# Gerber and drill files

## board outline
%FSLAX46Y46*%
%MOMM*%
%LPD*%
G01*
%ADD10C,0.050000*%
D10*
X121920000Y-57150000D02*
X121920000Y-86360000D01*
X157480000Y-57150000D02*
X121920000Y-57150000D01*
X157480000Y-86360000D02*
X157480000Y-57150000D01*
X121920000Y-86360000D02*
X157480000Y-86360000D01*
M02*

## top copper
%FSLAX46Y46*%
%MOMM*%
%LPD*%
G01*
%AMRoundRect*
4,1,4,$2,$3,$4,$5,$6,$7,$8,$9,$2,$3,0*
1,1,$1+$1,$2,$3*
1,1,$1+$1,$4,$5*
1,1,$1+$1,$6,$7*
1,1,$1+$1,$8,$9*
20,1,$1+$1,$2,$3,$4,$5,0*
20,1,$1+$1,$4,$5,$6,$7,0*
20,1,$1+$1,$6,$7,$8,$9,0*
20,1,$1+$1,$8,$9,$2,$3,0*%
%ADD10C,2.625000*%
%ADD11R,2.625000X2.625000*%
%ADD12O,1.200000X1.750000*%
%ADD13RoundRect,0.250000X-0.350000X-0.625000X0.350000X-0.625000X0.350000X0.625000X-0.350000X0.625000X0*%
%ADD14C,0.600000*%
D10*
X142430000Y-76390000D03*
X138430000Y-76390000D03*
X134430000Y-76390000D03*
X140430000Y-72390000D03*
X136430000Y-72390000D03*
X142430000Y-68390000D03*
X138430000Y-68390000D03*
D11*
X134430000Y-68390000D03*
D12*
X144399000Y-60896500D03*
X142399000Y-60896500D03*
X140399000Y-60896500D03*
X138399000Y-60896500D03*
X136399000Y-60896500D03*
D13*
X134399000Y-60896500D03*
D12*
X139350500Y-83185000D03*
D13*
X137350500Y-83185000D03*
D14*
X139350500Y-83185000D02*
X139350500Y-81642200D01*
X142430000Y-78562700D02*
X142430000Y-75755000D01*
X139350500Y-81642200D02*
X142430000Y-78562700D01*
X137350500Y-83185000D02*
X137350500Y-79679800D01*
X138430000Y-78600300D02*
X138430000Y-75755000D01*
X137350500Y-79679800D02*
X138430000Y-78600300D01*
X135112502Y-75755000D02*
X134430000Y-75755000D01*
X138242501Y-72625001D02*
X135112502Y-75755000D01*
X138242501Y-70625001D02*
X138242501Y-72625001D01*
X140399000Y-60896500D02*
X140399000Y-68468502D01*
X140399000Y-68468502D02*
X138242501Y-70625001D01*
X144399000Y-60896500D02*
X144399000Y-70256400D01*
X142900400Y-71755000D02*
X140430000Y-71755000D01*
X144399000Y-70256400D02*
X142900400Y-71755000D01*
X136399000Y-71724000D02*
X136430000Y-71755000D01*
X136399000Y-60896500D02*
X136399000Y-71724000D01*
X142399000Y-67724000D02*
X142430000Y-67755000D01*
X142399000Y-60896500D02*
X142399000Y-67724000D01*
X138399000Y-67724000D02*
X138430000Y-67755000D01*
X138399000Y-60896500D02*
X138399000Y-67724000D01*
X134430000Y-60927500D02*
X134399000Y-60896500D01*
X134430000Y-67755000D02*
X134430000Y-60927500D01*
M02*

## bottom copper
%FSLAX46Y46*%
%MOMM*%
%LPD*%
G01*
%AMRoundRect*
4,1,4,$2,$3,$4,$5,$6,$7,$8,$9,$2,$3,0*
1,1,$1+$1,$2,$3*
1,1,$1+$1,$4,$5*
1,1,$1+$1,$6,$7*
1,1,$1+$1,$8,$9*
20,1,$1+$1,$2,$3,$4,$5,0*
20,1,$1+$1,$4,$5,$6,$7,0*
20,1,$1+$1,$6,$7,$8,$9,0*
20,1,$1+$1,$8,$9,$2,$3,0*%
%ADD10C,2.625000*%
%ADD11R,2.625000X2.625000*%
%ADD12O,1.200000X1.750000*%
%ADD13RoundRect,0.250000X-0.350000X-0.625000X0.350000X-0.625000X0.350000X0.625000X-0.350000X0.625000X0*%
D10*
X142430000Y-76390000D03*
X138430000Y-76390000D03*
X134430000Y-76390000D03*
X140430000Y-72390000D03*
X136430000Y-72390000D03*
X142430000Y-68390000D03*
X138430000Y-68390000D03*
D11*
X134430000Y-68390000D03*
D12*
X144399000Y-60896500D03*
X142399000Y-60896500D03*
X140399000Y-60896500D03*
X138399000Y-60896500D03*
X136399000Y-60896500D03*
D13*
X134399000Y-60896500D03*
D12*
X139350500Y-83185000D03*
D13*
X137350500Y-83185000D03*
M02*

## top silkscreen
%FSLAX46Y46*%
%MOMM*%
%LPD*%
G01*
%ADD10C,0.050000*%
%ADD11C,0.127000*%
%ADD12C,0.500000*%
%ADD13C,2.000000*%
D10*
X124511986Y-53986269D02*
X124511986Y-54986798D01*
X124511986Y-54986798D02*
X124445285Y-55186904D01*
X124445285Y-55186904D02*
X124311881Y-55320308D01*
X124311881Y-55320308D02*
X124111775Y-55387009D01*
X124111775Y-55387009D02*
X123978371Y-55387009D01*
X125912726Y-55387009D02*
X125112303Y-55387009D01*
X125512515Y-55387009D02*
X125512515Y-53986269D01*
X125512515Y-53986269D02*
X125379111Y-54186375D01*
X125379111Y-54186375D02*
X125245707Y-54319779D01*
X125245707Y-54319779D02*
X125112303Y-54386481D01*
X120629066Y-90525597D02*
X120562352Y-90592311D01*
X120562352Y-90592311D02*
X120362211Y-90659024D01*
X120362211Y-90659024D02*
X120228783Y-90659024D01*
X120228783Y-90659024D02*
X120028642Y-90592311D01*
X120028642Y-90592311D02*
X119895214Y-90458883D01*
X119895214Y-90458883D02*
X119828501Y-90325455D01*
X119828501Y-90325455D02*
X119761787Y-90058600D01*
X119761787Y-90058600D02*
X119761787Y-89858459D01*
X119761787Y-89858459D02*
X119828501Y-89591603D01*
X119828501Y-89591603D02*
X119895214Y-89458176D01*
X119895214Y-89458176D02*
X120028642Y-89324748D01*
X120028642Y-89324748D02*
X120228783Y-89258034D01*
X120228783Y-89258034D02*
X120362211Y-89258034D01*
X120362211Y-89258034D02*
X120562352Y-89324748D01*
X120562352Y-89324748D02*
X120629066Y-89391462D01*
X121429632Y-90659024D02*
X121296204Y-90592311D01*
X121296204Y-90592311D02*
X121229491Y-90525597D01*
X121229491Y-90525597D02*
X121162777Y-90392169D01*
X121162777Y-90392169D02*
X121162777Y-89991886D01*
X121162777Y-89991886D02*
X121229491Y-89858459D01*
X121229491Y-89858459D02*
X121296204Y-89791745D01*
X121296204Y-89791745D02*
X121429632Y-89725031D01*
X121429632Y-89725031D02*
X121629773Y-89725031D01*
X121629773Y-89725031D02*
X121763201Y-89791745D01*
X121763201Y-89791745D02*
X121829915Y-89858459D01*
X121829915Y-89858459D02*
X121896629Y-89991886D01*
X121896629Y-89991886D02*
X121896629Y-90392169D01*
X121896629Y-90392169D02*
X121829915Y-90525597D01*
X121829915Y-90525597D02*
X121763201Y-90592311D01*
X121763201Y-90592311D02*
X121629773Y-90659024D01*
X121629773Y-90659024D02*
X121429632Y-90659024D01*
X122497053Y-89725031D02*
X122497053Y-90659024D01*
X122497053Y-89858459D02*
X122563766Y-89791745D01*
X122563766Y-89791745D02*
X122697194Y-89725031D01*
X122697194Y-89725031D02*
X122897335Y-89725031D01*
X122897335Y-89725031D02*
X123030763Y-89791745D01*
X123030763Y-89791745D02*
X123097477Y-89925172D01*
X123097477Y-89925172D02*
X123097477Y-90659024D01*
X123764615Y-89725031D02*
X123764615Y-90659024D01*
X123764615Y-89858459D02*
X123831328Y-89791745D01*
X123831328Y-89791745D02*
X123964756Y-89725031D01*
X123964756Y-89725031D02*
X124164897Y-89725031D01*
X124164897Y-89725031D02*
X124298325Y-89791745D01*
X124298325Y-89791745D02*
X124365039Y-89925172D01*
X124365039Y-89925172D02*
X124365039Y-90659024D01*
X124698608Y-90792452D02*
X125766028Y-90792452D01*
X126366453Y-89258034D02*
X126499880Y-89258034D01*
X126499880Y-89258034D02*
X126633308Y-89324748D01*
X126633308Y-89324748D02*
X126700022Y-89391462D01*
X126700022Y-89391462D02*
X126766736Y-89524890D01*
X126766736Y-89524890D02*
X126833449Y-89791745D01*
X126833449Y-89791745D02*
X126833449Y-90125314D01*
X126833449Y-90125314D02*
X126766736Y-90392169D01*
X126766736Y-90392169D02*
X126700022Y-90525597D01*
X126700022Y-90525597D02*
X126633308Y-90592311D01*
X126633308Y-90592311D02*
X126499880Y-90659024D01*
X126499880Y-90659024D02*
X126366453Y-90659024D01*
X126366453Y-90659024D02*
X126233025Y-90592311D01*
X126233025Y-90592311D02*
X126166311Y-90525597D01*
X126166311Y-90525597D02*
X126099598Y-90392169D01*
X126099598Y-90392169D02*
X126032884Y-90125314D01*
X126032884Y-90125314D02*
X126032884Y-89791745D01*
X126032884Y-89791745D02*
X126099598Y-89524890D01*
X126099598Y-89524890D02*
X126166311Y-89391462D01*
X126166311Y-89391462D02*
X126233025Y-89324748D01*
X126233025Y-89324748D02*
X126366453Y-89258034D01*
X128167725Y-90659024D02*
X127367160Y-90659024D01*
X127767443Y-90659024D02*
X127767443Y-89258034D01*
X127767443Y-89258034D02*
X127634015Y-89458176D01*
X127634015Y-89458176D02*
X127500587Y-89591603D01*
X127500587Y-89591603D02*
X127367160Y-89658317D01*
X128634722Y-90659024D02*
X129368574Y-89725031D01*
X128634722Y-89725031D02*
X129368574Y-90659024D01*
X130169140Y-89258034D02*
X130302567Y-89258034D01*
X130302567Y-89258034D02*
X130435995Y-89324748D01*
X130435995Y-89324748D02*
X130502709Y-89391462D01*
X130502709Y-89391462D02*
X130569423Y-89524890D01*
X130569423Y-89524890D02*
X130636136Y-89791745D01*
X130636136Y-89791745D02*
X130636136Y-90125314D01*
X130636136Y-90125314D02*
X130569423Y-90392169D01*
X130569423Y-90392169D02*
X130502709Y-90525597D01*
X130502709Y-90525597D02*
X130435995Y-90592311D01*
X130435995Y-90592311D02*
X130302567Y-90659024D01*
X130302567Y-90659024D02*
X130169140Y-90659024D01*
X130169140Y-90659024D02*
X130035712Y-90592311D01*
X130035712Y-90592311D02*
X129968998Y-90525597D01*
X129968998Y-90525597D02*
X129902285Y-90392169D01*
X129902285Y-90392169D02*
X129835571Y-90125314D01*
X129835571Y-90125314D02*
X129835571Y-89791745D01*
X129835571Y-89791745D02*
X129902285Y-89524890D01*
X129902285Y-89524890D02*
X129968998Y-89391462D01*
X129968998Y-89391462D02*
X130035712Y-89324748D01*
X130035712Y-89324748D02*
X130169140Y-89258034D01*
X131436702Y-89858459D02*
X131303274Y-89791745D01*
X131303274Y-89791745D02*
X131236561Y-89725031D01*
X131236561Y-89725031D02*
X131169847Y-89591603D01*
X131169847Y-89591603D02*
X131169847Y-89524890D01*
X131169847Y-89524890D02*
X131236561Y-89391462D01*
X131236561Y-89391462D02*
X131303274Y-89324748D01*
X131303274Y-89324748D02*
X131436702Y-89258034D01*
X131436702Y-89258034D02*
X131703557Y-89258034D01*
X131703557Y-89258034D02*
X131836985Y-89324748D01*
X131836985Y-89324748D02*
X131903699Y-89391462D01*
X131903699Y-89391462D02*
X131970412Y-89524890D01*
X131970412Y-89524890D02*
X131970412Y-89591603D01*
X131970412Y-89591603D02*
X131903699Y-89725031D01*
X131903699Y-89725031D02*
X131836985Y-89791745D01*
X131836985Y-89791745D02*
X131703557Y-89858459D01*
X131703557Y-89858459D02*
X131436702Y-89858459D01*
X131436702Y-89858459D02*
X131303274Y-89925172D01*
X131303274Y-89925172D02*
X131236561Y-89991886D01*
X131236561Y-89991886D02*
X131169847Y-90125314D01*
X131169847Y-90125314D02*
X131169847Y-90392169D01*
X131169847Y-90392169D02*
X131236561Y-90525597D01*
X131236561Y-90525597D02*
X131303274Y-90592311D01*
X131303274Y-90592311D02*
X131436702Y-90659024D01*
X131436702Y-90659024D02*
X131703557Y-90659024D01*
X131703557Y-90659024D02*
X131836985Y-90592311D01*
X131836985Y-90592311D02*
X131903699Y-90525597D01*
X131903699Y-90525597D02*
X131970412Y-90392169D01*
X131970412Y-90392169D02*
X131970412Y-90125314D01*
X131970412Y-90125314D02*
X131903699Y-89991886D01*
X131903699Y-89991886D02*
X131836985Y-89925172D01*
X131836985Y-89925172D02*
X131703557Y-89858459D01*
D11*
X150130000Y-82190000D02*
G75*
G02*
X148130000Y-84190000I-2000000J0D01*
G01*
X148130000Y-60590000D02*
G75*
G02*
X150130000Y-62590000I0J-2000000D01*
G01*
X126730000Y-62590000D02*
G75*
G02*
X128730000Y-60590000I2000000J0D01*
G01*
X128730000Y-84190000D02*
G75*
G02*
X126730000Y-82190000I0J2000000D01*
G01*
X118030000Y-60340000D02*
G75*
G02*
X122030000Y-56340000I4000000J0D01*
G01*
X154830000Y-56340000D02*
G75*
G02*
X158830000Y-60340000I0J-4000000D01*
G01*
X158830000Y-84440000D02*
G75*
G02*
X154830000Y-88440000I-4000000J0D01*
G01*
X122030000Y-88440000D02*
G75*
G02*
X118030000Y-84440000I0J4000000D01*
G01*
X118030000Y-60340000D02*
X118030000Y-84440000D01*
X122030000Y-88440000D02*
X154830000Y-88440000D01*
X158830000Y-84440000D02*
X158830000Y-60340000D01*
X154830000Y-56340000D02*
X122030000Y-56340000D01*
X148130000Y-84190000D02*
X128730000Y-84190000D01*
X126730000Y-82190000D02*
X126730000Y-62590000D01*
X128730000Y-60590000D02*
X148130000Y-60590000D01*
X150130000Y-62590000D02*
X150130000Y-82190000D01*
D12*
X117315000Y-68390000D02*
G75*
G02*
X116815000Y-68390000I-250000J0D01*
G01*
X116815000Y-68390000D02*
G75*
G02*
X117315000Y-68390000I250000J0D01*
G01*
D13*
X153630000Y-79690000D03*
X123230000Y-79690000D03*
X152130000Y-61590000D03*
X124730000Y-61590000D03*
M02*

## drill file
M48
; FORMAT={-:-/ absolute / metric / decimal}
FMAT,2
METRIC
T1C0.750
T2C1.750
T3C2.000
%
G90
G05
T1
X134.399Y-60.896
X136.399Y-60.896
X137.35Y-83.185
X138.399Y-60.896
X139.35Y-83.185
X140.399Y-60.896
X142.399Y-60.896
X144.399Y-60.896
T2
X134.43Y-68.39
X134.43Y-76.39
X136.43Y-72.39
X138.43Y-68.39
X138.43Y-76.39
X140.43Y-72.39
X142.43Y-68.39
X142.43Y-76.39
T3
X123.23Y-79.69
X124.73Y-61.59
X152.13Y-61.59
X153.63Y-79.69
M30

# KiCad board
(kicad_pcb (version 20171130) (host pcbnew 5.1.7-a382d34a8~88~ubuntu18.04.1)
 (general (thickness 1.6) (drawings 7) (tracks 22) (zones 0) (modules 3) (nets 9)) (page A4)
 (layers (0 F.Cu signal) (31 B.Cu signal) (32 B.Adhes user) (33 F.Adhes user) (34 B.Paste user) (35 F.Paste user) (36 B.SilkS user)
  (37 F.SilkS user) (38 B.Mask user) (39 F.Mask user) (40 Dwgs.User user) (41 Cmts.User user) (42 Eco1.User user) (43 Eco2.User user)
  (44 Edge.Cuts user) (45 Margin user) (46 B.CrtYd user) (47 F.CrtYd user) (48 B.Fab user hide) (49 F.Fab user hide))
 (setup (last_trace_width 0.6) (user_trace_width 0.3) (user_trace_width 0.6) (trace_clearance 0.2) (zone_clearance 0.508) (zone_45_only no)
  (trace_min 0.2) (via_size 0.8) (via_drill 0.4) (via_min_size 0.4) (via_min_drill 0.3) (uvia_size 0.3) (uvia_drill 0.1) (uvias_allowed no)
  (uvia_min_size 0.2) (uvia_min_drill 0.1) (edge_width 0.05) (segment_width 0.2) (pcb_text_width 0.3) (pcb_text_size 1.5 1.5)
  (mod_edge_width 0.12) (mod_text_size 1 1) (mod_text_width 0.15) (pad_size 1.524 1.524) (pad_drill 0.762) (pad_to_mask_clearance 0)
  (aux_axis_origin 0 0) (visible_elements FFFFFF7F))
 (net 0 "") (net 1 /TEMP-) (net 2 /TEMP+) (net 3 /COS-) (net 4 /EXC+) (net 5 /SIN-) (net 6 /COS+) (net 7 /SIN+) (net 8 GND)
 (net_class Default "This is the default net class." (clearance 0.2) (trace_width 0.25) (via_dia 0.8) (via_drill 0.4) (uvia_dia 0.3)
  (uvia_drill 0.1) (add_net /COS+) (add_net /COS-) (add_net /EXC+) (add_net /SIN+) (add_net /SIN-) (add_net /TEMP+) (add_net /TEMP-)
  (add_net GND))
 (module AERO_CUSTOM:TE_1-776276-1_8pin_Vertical (layer F.Cu) (at 138.43 72.39)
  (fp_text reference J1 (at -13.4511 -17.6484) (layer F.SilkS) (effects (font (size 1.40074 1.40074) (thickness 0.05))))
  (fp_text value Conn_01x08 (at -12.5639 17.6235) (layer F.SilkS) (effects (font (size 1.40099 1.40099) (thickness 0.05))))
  (fp_arc (start 9.7 9.8) (end 9.7 11.8) (angle -90) (layer F.SilkS) (width 0.127))
  (fp_arc (start 9.7 -9.8) (end 11.7 -9.8) (angle -90) (layer F.SilkS) (width 0.127))
  (fp_arc (start -9.7 -9.8) (end -9.7 -11.8) (angle -90) (layer F.SilkS) (width 0.127))
  (fp_arc (start -9.7 9.8) (end -11.7 9.8) (angle -90) (layer F.SilkS) (width 0.127))
  (fp_arc (start -16.4 -12.05) (end -20.4 -12.05) (angle 90) (layer F.SilkS) (width 0.127))
  (fp_arc (start 16.4 -12.05) (end 16.4 -16.05) (angle 90) (layer F.SilkS) (width 0.127))
  (fp_arc (start 16.4 12.05) (end 20.4 12.05) (angle 90) (layer F.SilkS) (width 0.127))
  (fp_arc (start -16.4 12.05) (end -16.4 16.05) (angle 90) (layer F.SilkS) (width 0.127))
  (fp_line (start -20.4 -12.05) (end -20.4 12.05) (layer F.SilkS) (width 0.127))
  (fp_line (start -16.4 16.05) (end 16.4 16.05) (layer F.SilkS) (width 0.127))
  (fp_line (start 20.4 12.05) (end 20.4 -12.05) (layer F.SilkS) (width 0.127))
  (fp_line (start 16.4 -16.05) (end -16.4 -16.05) (layer F.SilkS) (width 0.127))
  (fp_line (start 9.7 11.8) (end -9.7 11.8) (layer F.SilkS) (width 0.127))
  (fp_line (start -11.7 9.8) (end -11.7 -9.8) (layer F.SilkS) (width 0.127))
  (fp_line (start -9.7 -11.8) (end 9.7 -11.8) (layer F.SilkS) (width 0.127))
  (fp_line (start 11.7 -9.8) (end 11.7 9.8) (layer F.SilkS) (width 0.127))
  (fp_circle (center -21.365 -4) (end -21.115 -4) (layer F.SilkS) (width 0.5))
  (pad Hole np_thru_hole circle (at 15.2 7.3) (size 2 2) (drill 2) (layers *.Cu *.Mask F.SilkS))
  (pad Hole np_thru_hole circle (at -15.2 7.3) (size 2 2) (drill 2) (layers *.Cu *.Mask F.SilkS))
  (pad Hole np_thru_hole circle (at 13.7 -10.8) (size 2 2) (drill 2) (layers *.Cu *.Mask F.SilkS))
  (pad Hole np_thru_hole circle (at -13.7 -10.8) (size 2 2) (drill 2) (layers *.Cu *.Mask F.SilkS))
  (pad 8 thru_hole circle (at 4 4) (size 2.625 2.625) (drill 1.75) (layers *.Cu *.Mask) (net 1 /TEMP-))
  (pad 7 thru_hole circle (at 0 4) (size 2.625 2.625) (drill 1.75) (layers *.Cu *.Mask) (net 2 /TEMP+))
  (pad 6 thru_hole circle (at -4 4) (size 2.625 2.625) (drill 1.75) (layers *.Cu *.Mask) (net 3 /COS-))
  (pad 5 thru_hole circle (at 2 0) (size 2.625 2.625) (drill 1.75) (layers *.Cu *.Mask) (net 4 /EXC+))
  (pad 4 thru_hole circle (at -2 0) (size 2.625 2.625) (drill 1.75) (layers *.Cu *.Mask) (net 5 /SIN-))
  (pad 3 thru_hole circle (at 4 -4) (size 2.625 2.625) (drill 1.75) (layers *.Cu *.Mask) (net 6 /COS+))
  (pad 2 thru_hole circle (at 0 -4) (size 2.625 2.625) (drill 1.75) (layers *.Cu *.Mask) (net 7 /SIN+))
  (pad 1 thru_hole rect (at -4 -4) (size 2.625 2.625) (drill 1.75) (layers *.Cu *.Mask) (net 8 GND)))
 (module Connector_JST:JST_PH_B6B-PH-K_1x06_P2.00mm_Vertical (layer B.Cu) (at 134.399 60.8965)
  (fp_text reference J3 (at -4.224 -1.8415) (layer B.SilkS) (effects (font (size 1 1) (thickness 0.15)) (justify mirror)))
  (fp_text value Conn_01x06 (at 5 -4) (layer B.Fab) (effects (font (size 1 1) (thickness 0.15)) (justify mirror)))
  (pad 6 thru_hole oval (at 10 0) (size 1.2 1.75) (drill 0.75) (layers *.Cu *.Mask) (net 4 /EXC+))
  (pad 5 thru_hole oval (at 8 0) (size 1.2 1.75) (drill 0.75) (layers *.Cu *.Mask) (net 6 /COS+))
  (pad 4 thru_hole oval (at 6 0) (size 1.2 1.75) (drill 0.75) (layers *.Cu *.Mask) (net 3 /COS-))
  (pad 3 thru_hole oval (at 4 0) (size 1.2 1.75) (drill 0.75) (layers *.Cu *.Mask) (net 7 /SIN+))
  (pad 2 thru_hole oval (at 2 0) (size 1.2 1.75) (drill 0.75) (layers *.Cu *.Mask) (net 5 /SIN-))
  (pad 1 thru_hole roundrect (at 0 0) (size 1.2 1.75) (drill 0.75) (layers *.Cu *.Mask) (roundrect_rratio 0.208333) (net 8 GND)))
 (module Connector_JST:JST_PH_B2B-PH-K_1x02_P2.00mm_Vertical (layer B.Cu) (at 137.3505 83.185)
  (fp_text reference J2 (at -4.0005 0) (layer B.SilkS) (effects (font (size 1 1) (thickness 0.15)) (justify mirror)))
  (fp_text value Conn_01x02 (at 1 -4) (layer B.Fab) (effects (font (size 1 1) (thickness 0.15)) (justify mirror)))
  (pad 2 thru_hole oval (at 2 0) (size 1.2 1.75) (drill 0.75) (layers *.Cu *.Mask) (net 1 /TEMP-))
  (pad 1 thru_hole roundrect (at 0 0) (size 1.2 1.75) (drill 0.75) (layers *.Cu *.Mask) (roundrect_rratio 0.208333) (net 2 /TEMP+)))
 (gr_line (start 121.92 57.15) (end 121.92 86.36) (layer Edge.Cuts) (width 0.05))
 (gr_line (start 157.48 57.15) (end 121.92 57.15) (layer Edge.Cuts) (width 0.05))
 (gr_line (start 157.48 86.36) (end 157.48 57.15) (layer Edge.Cuts) (width 0.05))
 (gr_line (start 121.92 86.36) (end 157.48 86.36) (layer Edge.Cuts) (width 0.05))
 (segment (start 139.3505 83.185) (end 139.3505 81.6422) (width 0.6) (layer F.Cu) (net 1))
 (segment (start 142.43 78.5627) (end 142.43 75.755) (width 0.6) (layer F.Cu) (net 1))
 (segment (start 139.3505 81.6422) (end 142.43 78.5627) (width 0.6) (layer F.Cu) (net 1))
 (segment (start 137.3505 83.185) (end 137.3505 79.6798) (width 0.6) (layer F.Cu) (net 2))
 (segment (start 138.43 78.6003) (end 138.43 75.755) (width 0.6) (layer F.Cu) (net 2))
 (segment (start 137.3505 79.6798) (end 138.43 78.6003) (width 0.6) (layer F.Cu) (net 2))
 (segment (start 135.112502 75.755) (end 134.43 75.755) (width 0.6) (layer F.Cu) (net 3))
 (segment (start 138.242501 72.625001) (end 135.112502 75.755) (width 0.6) (layer F.Cu) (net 3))
 (segment (start 138.242501 70.625001) (end 138.242501 72.625001) (width 0.6) (layer F.Cu) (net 3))
 (segment (start 140.399 60.8965) (end 140.399 68.468502) (width 0.6) (layer F.Cu) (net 3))
 (segment (start 140.399 68.468502) (end 138.242501 70.625001) (width 0.6) (layer F.Cu) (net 3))
 (segment (start 144.399 60.8965) (end 144.399 70.2564) (width 0.6) (layer F.Cu) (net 4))
 (segment (start 142.9004 71.755) (end 140.43 71.755) (width 0.6) (layer F.Cu) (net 4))
 (segment (start 144.399 70.2564) (end 142.9004 71.755) (width 0.6) (layer F.Cu) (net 4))
 (segment (start 136.399 71.724) (end 136.43 71.755) (width 0.6) (layer F.Cu) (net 5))
 (segment (start 136.399 60.8965) (end 136.399 71.724) (width 0.6) (layer F.Cu) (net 5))
 (segment (start 142.399 67.724) (end 142.43 67.755) (width 0.6) (layer F.Cu) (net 6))
 (segment (start 142.399 60.8965) (end 142.399 67.724) (width 0.6) (layer F.Cu) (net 6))
 (segment (start 138.399 67.724) (end 138.43 67.755) (width 0.6) (layer F.Cu) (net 7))
 (segment (start 138.399 60.8965) (end 138.399 67.724) (width 0.6) (layer F.Cu) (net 7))
 (segment (start 134.43 60.9275) (end 134.399 60.8965) (width 0.6) (layer F.Cu) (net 8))
 (segment (start 134.43 67.755) (end 134.43 60.9275) (width 0.6) (layer F.Cu) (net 8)))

